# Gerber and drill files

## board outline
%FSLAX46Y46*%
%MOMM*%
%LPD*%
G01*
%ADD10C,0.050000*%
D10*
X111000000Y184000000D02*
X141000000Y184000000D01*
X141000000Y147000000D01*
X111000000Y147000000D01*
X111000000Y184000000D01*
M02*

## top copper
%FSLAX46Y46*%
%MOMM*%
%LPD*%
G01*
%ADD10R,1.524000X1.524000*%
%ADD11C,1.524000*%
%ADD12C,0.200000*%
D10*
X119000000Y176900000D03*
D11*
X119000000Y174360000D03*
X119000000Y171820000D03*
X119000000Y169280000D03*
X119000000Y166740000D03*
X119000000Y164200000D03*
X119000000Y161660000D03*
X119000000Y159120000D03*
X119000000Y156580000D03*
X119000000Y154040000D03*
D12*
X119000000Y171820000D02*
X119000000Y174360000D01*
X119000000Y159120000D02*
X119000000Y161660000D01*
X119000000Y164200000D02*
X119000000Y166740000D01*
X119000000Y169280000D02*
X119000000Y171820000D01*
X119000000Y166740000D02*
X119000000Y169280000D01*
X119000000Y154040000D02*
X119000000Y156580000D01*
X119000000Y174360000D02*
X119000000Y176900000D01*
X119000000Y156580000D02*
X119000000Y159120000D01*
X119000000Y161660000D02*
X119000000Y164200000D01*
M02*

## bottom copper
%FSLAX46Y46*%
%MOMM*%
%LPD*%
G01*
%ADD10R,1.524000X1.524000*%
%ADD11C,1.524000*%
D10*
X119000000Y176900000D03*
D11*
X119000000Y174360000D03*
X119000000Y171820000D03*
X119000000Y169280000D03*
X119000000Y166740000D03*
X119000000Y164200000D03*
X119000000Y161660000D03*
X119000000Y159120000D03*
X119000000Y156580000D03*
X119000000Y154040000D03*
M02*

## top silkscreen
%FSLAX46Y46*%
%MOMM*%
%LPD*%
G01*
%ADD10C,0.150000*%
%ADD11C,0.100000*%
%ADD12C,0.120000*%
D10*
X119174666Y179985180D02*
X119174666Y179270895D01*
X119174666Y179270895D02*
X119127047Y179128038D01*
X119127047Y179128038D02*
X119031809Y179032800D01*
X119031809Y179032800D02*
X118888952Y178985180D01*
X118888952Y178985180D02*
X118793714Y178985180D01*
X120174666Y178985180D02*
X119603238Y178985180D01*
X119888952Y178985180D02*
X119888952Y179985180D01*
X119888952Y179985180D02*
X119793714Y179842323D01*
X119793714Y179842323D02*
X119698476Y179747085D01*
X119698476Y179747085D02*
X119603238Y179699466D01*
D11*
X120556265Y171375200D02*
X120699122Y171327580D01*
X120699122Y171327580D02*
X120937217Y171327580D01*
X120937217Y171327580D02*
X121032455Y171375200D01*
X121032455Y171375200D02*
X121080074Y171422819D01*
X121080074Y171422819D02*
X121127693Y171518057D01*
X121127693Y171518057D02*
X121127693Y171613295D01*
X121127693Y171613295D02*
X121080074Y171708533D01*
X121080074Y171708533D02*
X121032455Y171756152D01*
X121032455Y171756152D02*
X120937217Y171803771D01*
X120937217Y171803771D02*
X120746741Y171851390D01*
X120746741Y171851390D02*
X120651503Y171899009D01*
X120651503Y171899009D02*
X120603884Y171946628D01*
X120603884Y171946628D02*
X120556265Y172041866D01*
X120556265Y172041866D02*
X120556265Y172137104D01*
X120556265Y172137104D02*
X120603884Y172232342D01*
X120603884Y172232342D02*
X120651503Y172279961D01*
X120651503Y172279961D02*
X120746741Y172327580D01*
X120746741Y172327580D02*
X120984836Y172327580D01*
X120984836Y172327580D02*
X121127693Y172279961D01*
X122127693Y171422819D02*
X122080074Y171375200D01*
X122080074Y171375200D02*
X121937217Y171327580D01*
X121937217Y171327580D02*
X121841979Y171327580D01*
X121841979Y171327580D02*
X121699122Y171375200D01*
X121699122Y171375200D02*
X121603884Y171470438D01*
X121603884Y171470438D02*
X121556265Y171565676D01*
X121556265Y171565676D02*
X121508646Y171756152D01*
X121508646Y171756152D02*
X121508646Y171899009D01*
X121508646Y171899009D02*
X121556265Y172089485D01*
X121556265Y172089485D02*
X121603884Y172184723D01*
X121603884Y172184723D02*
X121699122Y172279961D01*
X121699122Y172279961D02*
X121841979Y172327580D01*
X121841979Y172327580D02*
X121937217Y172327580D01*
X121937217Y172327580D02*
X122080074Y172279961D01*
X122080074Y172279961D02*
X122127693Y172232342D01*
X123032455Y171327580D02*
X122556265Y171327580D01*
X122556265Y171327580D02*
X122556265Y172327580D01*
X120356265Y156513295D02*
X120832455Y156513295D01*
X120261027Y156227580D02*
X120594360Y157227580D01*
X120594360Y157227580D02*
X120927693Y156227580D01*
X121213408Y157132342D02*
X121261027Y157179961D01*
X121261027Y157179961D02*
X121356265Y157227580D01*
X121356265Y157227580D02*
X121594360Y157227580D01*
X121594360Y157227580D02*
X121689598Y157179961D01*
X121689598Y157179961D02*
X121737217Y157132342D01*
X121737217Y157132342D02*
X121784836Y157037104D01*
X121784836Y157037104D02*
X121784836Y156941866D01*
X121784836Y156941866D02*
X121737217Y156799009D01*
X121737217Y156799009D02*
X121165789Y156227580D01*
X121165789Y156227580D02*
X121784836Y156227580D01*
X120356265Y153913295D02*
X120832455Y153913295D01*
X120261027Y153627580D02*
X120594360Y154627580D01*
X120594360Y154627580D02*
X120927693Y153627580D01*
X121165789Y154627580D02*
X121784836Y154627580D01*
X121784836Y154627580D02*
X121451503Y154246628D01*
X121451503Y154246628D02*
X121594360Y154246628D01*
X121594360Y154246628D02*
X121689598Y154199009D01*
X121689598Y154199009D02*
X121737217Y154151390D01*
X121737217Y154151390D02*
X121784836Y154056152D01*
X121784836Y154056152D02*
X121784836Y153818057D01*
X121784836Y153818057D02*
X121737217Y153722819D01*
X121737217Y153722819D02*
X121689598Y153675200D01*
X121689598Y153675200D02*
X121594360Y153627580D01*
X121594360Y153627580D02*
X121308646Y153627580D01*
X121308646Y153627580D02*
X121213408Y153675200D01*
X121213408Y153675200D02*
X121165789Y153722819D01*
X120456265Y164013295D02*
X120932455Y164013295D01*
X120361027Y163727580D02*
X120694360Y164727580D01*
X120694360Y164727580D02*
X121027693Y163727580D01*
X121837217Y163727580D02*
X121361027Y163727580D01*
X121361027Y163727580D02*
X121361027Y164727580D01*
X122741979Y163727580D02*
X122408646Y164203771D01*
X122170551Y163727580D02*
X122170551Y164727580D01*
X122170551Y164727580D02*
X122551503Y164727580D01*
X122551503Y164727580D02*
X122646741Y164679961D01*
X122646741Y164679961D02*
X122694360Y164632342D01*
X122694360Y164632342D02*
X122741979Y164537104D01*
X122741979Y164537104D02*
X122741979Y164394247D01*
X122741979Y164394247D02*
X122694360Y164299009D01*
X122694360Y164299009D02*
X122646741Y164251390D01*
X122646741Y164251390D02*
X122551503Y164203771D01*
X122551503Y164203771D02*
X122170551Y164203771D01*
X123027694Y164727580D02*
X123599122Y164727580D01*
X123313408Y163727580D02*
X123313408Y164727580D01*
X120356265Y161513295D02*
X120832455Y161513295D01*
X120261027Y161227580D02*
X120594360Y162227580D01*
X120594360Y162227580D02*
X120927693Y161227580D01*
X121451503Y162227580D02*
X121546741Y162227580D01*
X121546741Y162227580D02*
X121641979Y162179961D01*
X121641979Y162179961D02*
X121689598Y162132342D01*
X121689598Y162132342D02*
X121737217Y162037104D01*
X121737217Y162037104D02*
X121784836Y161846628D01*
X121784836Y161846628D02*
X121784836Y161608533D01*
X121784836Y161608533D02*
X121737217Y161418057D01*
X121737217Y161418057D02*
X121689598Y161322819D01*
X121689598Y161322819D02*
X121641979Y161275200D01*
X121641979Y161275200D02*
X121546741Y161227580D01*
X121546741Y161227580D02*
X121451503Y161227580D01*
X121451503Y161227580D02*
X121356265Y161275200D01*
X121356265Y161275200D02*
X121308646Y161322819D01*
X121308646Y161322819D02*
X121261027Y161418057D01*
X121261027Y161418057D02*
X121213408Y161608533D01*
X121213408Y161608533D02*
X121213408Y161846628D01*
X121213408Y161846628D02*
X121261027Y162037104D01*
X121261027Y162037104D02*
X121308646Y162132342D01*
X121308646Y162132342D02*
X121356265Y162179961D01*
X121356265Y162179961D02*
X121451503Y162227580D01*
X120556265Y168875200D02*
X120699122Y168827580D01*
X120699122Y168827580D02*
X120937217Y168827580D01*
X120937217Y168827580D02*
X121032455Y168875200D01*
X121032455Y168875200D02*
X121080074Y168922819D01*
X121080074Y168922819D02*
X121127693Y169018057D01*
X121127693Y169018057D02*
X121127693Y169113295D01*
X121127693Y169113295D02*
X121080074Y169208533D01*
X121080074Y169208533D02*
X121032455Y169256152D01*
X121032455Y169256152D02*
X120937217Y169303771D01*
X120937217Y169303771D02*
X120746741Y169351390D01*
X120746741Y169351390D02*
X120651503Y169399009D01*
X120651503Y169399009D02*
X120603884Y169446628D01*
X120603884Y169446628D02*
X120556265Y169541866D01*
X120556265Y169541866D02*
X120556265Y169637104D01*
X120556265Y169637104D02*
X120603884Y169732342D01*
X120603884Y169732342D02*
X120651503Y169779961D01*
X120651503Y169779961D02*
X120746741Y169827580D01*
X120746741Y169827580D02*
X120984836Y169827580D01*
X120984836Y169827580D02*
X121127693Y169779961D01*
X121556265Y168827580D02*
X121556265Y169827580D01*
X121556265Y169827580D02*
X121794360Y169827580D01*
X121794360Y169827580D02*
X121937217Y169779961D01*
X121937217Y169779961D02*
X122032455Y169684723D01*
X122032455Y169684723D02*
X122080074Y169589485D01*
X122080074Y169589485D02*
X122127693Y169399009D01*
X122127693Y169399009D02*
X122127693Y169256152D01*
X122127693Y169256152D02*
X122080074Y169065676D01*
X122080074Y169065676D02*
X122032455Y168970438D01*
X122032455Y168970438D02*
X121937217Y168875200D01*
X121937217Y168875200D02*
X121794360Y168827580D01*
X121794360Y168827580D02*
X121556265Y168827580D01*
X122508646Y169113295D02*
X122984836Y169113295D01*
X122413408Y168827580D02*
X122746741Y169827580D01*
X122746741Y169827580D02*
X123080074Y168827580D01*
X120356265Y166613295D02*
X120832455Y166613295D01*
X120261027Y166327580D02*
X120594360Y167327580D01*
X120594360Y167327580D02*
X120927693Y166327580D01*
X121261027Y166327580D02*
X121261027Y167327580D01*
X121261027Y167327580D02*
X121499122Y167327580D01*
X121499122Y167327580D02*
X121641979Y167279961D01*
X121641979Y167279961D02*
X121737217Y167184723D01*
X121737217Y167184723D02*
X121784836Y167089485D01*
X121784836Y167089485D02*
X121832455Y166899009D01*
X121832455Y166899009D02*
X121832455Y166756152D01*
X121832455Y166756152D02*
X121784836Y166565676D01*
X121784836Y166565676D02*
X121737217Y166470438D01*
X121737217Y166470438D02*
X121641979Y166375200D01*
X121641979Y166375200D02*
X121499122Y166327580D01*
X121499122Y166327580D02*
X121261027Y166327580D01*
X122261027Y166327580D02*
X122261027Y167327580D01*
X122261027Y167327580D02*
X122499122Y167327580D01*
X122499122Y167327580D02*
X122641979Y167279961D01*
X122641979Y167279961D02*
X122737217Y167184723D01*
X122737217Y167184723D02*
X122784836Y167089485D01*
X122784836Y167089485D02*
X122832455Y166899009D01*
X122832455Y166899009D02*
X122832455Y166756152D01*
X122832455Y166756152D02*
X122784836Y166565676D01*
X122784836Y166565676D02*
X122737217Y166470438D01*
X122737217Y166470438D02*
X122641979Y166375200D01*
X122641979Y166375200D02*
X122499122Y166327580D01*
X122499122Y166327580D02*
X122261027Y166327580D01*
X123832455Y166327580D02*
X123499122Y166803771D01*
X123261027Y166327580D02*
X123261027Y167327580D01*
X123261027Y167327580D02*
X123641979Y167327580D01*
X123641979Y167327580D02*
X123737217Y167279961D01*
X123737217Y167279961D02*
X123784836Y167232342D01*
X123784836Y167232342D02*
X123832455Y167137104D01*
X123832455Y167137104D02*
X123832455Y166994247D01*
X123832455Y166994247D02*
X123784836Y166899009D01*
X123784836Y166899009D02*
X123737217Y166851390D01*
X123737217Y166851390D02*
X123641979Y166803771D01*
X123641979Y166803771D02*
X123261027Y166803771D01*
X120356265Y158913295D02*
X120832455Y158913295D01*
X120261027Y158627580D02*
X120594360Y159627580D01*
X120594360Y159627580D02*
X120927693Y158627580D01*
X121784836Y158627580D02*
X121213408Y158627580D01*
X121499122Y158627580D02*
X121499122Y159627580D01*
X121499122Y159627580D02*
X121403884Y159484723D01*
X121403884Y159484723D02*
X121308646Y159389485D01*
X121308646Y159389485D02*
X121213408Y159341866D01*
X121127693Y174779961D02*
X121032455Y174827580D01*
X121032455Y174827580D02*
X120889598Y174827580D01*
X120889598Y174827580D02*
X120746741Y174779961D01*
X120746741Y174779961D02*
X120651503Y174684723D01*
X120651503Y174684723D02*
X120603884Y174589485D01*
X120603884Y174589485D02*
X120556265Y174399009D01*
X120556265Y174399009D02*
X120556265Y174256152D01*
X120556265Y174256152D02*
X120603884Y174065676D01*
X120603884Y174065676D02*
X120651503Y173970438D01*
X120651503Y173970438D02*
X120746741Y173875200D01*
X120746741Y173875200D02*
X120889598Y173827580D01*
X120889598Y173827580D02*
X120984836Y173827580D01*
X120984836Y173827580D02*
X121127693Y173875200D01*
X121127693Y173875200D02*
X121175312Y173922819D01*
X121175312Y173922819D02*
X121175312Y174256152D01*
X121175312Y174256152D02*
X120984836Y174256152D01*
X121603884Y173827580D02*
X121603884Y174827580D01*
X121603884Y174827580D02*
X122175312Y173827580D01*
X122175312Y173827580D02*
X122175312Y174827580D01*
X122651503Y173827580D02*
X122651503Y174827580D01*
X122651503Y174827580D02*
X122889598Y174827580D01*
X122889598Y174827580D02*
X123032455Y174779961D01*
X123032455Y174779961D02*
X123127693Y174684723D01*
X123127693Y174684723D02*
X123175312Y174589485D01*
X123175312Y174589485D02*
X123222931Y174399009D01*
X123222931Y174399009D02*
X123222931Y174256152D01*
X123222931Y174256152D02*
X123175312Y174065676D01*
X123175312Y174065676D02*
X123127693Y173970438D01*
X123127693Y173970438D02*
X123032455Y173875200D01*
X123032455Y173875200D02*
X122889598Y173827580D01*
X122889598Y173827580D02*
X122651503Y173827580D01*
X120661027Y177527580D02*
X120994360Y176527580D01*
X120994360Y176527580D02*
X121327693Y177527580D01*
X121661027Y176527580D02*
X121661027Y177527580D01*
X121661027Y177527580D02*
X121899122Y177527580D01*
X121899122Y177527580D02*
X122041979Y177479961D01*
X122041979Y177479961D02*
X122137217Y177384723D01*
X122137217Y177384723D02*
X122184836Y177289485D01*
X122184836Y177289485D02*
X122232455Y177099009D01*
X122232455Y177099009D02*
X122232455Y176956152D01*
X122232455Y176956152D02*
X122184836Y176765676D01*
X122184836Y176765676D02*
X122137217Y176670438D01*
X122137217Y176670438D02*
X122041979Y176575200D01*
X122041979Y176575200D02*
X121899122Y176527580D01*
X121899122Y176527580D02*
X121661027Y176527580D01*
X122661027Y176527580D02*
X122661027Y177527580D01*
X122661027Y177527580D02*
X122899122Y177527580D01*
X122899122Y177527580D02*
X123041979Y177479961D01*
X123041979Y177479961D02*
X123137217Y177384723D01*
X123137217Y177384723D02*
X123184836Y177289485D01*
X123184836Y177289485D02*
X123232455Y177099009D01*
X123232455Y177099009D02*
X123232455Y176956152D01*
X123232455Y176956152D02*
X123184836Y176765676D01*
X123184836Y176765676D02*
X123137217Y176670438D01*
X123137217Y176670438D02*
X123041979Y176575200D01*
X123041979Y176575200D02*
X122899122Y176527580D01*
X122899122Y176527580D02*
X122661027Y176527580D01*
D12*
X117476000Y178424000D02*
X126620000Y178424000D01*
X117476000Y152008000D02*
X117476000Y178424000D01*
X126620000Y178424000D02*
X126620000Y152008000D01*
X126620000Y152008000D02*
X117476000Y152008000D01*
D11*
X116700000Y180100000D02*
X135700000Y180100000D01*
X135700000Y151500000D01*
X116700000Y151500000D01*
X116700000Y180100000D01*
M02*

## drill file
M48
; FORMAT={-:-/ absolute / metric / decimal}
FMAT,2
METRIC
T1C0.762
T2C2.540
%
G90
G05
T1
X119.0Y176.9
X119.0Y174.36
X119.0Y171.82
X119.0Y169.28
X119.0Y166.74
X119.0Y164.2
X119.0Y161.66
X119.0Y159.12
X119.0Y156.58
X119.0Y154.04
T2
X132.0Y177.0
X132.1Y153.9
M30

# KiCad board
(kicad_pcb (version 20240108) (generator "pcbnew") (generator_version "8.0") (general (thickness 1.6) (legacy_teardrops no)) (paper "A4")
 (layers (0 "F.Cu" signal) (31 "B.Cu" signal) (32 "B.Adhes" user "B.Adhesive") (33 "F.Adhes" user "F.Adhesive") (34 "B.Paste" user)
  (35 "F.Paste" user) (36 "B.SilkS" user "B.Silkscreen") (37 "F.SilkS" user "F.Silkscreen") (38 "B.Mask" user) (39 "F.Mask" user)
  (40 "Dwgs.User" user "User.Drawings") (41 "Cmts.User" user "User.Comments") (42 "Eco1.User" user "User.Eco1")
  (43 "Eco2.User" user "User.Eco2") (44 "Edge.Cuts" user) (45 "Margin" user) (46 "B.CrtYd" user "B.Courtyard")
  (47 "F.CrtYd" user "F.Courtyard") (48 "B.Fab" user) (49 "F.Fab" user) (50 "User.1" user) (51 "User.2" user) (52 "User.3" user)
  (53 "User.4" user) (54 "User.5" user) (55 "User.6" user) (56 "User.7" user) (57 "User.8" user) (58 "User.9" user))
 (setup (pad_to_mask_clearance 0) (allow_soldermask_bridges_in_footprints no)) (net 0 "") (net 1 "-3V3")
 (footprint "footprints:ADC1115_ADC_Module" (layer "F.Cu") (at 119 -176.9)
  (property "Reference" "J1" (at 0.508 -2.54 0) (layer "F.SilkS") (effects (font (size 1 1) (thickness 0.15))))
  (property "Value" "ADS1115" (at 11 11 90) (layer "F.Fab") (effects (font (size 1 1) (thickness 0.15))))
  (fp_line (start -1.524 -1.524) (end 7.62 -1.524) (stroke (width 0.12) (type solid)) (layer "F.SilkS"))
  (fp_line (start -1.524 24.892) (end -1.524 -1.524) (stroke (width 0.12) (type solid)) (layer "F.SilkS"))
  (fp_line (start 7.62 -1.524) (end 7.62 24.892) (stroke (width 0.12) (type solid)) (layer "F.SilkS"))
  (fp_line (start 7.62 24.892) (end -1.524 24.892) (stroke (width 0.12) (type solid)) (layer "F.SilkS"))
  (fp_rect (start -2.3 -3.2) (end 16.7 25.4) (stroke (width 0.1) (type default)) (fill none) (layer "F.SilkS"))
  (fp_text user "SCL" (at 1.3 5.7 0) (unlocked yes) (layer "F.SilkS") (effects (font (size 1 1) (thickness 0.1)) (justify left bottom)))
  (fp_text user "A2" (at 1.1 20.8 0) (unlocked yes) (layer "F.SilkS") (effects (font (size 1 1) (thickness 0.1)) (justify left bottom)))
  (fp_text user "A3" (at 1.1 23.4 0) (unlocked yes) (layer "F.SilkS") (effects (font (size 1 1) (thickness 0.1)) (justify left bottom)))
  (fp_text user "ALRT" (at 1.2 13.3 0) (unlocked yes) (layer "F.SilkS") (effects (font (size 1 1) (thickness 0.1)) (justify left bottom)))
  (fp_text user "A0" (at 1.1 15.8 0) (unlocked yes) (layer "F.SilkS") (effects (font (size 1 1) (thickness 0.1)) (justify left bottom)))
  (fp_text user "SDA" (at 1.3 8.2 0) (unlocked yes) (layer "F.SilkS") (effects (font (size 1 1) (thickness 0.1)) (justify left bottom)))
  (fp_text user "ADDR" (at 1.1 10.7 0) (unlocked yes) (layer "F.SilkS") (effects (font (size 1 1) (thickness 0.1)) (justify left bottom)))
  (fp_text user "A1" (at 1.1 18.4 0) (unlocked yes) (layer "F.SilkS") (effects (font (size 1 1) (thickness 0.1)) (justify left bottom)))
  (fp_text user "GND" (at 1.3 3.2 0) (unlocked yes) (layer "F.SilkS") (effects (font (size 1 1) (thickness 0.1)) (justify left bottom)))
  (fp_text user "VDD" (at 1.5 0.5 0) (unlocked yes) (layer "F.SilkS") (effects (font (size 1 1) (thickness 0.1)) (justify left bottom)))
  (pad "" np_thru_hole circle (at 13 -0.1) (size 2.54 2.54) (drill 2.54) (layers "F&B.Cu" "*.Mask"))
  (pad "" np_thru_hole circle (at 13.1 23) (size 2.54 2.54) (drill 2.54) (layers "F&B.Cu" "*.Mask"))
  (pad "1" thru_hole rect (at 0 0) (size 1.524 1.524) (drill 0.762) (layers "*.Cu" "*.Mask") (remove_unused_layers no) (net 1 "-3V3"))
  (pad "2" thru_hole circle (at 0 2.54) (size 1.524 1.524) (drill 0.762) (layers "*.Cu" "*.Mask") (remove_unused_layers no) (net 1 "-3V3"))
  (pad "3" thru_hole circle (at 0 5.08) (size 1.524 1.524) (drill 0.762) (layers "*.Cu" "*.Mask") (remove_unused_layers no) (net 1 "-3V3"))
  (pad "4" thru_hole circle (at 0 7.62) (size 1.524 1.524) (drill 0.762) (layers "*.Cu" "*.Mask") (remove_unused_layers no) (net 1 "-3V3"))
  (pad "5" thru_hole circle (at 0 10.16) (size 1.524 1.524) (drill 0.762) (layers "*.Cu" "*.Mask") (remove_unused_layers no) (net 1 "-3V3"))
  (pad "6" thru_hole circle (at 0 12.7) (size 1.524 1.524) (drill 0.762) (layers "*.Cu" "*.Mask") (remove_unused_layers no) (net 1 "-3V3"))
  (pad "7" thru_hole circle (at 0 15.24) (size 1.524 1.524) (drill 0.762) (layers "*.Cu" "*.Mask") (remove_unused_layers no) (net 1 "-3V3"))
  (pad "8" thru_hole circle (at 0 17.78) (size 1.524 1.524) (drill 0.762) (layers "*.Cu" "*.Mask") (remove_unused_layers no) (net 1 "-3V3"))
  (pad "9" thru_hole circle (at 0 20.32) (size 1.524 1.524) (drill 0.762) (layers "*.Cu" "*.Mask") (remove_unused_layers no) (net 1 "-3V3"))
  (pad "10" thru_hole circle (at 0 22.86) (size 1.524 1.524) (drill 0.762) (layers "*.Cu" "*.Mask") (remove_unused_layers no) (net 1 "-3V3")))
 (gr_rect (start 111 -184) (end 141 -147) (stroke (width 0.05) (type default)) (fill none) (layer "Edge.Cuts"))
 (segment (start 119 -171.82) (end 119 -174.36) (width 0.2) (layer "F.Cu") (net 1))
 (segment (start 119 -159.12) (end 119 -161.66) (width 0.2) (layer "F.Cu") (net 1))
 (segment (start 119 -164.2) (end 119 -166.74) (width 0.2) (layer "F.Cu") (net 1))
 (segment (start 119 -169.28) (end 119 -171.82) (width 0.2) (layer "F.Cu") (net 1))
 (segment (start 119 -166.74) (end 119 -169.28) (width 0.2) (layer "F.Cu") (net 1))
 (segment (start 119 -154.04) (end 119 -156.58) (width 0.2) (layer "F.Cu") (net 1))
 (segment (start 119 -174.36) (end 119 -176.9) (width 0.2) (layer "F.Cu") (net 1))
 (segment (start 119 -156.58) (end 119 -159.12) (width 0.2) (layer "F.Cu") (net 1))
 (segment (start 119 -161.66) (end 119 -164.2) (width 0.2) (layer "F.Cu") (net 1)))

